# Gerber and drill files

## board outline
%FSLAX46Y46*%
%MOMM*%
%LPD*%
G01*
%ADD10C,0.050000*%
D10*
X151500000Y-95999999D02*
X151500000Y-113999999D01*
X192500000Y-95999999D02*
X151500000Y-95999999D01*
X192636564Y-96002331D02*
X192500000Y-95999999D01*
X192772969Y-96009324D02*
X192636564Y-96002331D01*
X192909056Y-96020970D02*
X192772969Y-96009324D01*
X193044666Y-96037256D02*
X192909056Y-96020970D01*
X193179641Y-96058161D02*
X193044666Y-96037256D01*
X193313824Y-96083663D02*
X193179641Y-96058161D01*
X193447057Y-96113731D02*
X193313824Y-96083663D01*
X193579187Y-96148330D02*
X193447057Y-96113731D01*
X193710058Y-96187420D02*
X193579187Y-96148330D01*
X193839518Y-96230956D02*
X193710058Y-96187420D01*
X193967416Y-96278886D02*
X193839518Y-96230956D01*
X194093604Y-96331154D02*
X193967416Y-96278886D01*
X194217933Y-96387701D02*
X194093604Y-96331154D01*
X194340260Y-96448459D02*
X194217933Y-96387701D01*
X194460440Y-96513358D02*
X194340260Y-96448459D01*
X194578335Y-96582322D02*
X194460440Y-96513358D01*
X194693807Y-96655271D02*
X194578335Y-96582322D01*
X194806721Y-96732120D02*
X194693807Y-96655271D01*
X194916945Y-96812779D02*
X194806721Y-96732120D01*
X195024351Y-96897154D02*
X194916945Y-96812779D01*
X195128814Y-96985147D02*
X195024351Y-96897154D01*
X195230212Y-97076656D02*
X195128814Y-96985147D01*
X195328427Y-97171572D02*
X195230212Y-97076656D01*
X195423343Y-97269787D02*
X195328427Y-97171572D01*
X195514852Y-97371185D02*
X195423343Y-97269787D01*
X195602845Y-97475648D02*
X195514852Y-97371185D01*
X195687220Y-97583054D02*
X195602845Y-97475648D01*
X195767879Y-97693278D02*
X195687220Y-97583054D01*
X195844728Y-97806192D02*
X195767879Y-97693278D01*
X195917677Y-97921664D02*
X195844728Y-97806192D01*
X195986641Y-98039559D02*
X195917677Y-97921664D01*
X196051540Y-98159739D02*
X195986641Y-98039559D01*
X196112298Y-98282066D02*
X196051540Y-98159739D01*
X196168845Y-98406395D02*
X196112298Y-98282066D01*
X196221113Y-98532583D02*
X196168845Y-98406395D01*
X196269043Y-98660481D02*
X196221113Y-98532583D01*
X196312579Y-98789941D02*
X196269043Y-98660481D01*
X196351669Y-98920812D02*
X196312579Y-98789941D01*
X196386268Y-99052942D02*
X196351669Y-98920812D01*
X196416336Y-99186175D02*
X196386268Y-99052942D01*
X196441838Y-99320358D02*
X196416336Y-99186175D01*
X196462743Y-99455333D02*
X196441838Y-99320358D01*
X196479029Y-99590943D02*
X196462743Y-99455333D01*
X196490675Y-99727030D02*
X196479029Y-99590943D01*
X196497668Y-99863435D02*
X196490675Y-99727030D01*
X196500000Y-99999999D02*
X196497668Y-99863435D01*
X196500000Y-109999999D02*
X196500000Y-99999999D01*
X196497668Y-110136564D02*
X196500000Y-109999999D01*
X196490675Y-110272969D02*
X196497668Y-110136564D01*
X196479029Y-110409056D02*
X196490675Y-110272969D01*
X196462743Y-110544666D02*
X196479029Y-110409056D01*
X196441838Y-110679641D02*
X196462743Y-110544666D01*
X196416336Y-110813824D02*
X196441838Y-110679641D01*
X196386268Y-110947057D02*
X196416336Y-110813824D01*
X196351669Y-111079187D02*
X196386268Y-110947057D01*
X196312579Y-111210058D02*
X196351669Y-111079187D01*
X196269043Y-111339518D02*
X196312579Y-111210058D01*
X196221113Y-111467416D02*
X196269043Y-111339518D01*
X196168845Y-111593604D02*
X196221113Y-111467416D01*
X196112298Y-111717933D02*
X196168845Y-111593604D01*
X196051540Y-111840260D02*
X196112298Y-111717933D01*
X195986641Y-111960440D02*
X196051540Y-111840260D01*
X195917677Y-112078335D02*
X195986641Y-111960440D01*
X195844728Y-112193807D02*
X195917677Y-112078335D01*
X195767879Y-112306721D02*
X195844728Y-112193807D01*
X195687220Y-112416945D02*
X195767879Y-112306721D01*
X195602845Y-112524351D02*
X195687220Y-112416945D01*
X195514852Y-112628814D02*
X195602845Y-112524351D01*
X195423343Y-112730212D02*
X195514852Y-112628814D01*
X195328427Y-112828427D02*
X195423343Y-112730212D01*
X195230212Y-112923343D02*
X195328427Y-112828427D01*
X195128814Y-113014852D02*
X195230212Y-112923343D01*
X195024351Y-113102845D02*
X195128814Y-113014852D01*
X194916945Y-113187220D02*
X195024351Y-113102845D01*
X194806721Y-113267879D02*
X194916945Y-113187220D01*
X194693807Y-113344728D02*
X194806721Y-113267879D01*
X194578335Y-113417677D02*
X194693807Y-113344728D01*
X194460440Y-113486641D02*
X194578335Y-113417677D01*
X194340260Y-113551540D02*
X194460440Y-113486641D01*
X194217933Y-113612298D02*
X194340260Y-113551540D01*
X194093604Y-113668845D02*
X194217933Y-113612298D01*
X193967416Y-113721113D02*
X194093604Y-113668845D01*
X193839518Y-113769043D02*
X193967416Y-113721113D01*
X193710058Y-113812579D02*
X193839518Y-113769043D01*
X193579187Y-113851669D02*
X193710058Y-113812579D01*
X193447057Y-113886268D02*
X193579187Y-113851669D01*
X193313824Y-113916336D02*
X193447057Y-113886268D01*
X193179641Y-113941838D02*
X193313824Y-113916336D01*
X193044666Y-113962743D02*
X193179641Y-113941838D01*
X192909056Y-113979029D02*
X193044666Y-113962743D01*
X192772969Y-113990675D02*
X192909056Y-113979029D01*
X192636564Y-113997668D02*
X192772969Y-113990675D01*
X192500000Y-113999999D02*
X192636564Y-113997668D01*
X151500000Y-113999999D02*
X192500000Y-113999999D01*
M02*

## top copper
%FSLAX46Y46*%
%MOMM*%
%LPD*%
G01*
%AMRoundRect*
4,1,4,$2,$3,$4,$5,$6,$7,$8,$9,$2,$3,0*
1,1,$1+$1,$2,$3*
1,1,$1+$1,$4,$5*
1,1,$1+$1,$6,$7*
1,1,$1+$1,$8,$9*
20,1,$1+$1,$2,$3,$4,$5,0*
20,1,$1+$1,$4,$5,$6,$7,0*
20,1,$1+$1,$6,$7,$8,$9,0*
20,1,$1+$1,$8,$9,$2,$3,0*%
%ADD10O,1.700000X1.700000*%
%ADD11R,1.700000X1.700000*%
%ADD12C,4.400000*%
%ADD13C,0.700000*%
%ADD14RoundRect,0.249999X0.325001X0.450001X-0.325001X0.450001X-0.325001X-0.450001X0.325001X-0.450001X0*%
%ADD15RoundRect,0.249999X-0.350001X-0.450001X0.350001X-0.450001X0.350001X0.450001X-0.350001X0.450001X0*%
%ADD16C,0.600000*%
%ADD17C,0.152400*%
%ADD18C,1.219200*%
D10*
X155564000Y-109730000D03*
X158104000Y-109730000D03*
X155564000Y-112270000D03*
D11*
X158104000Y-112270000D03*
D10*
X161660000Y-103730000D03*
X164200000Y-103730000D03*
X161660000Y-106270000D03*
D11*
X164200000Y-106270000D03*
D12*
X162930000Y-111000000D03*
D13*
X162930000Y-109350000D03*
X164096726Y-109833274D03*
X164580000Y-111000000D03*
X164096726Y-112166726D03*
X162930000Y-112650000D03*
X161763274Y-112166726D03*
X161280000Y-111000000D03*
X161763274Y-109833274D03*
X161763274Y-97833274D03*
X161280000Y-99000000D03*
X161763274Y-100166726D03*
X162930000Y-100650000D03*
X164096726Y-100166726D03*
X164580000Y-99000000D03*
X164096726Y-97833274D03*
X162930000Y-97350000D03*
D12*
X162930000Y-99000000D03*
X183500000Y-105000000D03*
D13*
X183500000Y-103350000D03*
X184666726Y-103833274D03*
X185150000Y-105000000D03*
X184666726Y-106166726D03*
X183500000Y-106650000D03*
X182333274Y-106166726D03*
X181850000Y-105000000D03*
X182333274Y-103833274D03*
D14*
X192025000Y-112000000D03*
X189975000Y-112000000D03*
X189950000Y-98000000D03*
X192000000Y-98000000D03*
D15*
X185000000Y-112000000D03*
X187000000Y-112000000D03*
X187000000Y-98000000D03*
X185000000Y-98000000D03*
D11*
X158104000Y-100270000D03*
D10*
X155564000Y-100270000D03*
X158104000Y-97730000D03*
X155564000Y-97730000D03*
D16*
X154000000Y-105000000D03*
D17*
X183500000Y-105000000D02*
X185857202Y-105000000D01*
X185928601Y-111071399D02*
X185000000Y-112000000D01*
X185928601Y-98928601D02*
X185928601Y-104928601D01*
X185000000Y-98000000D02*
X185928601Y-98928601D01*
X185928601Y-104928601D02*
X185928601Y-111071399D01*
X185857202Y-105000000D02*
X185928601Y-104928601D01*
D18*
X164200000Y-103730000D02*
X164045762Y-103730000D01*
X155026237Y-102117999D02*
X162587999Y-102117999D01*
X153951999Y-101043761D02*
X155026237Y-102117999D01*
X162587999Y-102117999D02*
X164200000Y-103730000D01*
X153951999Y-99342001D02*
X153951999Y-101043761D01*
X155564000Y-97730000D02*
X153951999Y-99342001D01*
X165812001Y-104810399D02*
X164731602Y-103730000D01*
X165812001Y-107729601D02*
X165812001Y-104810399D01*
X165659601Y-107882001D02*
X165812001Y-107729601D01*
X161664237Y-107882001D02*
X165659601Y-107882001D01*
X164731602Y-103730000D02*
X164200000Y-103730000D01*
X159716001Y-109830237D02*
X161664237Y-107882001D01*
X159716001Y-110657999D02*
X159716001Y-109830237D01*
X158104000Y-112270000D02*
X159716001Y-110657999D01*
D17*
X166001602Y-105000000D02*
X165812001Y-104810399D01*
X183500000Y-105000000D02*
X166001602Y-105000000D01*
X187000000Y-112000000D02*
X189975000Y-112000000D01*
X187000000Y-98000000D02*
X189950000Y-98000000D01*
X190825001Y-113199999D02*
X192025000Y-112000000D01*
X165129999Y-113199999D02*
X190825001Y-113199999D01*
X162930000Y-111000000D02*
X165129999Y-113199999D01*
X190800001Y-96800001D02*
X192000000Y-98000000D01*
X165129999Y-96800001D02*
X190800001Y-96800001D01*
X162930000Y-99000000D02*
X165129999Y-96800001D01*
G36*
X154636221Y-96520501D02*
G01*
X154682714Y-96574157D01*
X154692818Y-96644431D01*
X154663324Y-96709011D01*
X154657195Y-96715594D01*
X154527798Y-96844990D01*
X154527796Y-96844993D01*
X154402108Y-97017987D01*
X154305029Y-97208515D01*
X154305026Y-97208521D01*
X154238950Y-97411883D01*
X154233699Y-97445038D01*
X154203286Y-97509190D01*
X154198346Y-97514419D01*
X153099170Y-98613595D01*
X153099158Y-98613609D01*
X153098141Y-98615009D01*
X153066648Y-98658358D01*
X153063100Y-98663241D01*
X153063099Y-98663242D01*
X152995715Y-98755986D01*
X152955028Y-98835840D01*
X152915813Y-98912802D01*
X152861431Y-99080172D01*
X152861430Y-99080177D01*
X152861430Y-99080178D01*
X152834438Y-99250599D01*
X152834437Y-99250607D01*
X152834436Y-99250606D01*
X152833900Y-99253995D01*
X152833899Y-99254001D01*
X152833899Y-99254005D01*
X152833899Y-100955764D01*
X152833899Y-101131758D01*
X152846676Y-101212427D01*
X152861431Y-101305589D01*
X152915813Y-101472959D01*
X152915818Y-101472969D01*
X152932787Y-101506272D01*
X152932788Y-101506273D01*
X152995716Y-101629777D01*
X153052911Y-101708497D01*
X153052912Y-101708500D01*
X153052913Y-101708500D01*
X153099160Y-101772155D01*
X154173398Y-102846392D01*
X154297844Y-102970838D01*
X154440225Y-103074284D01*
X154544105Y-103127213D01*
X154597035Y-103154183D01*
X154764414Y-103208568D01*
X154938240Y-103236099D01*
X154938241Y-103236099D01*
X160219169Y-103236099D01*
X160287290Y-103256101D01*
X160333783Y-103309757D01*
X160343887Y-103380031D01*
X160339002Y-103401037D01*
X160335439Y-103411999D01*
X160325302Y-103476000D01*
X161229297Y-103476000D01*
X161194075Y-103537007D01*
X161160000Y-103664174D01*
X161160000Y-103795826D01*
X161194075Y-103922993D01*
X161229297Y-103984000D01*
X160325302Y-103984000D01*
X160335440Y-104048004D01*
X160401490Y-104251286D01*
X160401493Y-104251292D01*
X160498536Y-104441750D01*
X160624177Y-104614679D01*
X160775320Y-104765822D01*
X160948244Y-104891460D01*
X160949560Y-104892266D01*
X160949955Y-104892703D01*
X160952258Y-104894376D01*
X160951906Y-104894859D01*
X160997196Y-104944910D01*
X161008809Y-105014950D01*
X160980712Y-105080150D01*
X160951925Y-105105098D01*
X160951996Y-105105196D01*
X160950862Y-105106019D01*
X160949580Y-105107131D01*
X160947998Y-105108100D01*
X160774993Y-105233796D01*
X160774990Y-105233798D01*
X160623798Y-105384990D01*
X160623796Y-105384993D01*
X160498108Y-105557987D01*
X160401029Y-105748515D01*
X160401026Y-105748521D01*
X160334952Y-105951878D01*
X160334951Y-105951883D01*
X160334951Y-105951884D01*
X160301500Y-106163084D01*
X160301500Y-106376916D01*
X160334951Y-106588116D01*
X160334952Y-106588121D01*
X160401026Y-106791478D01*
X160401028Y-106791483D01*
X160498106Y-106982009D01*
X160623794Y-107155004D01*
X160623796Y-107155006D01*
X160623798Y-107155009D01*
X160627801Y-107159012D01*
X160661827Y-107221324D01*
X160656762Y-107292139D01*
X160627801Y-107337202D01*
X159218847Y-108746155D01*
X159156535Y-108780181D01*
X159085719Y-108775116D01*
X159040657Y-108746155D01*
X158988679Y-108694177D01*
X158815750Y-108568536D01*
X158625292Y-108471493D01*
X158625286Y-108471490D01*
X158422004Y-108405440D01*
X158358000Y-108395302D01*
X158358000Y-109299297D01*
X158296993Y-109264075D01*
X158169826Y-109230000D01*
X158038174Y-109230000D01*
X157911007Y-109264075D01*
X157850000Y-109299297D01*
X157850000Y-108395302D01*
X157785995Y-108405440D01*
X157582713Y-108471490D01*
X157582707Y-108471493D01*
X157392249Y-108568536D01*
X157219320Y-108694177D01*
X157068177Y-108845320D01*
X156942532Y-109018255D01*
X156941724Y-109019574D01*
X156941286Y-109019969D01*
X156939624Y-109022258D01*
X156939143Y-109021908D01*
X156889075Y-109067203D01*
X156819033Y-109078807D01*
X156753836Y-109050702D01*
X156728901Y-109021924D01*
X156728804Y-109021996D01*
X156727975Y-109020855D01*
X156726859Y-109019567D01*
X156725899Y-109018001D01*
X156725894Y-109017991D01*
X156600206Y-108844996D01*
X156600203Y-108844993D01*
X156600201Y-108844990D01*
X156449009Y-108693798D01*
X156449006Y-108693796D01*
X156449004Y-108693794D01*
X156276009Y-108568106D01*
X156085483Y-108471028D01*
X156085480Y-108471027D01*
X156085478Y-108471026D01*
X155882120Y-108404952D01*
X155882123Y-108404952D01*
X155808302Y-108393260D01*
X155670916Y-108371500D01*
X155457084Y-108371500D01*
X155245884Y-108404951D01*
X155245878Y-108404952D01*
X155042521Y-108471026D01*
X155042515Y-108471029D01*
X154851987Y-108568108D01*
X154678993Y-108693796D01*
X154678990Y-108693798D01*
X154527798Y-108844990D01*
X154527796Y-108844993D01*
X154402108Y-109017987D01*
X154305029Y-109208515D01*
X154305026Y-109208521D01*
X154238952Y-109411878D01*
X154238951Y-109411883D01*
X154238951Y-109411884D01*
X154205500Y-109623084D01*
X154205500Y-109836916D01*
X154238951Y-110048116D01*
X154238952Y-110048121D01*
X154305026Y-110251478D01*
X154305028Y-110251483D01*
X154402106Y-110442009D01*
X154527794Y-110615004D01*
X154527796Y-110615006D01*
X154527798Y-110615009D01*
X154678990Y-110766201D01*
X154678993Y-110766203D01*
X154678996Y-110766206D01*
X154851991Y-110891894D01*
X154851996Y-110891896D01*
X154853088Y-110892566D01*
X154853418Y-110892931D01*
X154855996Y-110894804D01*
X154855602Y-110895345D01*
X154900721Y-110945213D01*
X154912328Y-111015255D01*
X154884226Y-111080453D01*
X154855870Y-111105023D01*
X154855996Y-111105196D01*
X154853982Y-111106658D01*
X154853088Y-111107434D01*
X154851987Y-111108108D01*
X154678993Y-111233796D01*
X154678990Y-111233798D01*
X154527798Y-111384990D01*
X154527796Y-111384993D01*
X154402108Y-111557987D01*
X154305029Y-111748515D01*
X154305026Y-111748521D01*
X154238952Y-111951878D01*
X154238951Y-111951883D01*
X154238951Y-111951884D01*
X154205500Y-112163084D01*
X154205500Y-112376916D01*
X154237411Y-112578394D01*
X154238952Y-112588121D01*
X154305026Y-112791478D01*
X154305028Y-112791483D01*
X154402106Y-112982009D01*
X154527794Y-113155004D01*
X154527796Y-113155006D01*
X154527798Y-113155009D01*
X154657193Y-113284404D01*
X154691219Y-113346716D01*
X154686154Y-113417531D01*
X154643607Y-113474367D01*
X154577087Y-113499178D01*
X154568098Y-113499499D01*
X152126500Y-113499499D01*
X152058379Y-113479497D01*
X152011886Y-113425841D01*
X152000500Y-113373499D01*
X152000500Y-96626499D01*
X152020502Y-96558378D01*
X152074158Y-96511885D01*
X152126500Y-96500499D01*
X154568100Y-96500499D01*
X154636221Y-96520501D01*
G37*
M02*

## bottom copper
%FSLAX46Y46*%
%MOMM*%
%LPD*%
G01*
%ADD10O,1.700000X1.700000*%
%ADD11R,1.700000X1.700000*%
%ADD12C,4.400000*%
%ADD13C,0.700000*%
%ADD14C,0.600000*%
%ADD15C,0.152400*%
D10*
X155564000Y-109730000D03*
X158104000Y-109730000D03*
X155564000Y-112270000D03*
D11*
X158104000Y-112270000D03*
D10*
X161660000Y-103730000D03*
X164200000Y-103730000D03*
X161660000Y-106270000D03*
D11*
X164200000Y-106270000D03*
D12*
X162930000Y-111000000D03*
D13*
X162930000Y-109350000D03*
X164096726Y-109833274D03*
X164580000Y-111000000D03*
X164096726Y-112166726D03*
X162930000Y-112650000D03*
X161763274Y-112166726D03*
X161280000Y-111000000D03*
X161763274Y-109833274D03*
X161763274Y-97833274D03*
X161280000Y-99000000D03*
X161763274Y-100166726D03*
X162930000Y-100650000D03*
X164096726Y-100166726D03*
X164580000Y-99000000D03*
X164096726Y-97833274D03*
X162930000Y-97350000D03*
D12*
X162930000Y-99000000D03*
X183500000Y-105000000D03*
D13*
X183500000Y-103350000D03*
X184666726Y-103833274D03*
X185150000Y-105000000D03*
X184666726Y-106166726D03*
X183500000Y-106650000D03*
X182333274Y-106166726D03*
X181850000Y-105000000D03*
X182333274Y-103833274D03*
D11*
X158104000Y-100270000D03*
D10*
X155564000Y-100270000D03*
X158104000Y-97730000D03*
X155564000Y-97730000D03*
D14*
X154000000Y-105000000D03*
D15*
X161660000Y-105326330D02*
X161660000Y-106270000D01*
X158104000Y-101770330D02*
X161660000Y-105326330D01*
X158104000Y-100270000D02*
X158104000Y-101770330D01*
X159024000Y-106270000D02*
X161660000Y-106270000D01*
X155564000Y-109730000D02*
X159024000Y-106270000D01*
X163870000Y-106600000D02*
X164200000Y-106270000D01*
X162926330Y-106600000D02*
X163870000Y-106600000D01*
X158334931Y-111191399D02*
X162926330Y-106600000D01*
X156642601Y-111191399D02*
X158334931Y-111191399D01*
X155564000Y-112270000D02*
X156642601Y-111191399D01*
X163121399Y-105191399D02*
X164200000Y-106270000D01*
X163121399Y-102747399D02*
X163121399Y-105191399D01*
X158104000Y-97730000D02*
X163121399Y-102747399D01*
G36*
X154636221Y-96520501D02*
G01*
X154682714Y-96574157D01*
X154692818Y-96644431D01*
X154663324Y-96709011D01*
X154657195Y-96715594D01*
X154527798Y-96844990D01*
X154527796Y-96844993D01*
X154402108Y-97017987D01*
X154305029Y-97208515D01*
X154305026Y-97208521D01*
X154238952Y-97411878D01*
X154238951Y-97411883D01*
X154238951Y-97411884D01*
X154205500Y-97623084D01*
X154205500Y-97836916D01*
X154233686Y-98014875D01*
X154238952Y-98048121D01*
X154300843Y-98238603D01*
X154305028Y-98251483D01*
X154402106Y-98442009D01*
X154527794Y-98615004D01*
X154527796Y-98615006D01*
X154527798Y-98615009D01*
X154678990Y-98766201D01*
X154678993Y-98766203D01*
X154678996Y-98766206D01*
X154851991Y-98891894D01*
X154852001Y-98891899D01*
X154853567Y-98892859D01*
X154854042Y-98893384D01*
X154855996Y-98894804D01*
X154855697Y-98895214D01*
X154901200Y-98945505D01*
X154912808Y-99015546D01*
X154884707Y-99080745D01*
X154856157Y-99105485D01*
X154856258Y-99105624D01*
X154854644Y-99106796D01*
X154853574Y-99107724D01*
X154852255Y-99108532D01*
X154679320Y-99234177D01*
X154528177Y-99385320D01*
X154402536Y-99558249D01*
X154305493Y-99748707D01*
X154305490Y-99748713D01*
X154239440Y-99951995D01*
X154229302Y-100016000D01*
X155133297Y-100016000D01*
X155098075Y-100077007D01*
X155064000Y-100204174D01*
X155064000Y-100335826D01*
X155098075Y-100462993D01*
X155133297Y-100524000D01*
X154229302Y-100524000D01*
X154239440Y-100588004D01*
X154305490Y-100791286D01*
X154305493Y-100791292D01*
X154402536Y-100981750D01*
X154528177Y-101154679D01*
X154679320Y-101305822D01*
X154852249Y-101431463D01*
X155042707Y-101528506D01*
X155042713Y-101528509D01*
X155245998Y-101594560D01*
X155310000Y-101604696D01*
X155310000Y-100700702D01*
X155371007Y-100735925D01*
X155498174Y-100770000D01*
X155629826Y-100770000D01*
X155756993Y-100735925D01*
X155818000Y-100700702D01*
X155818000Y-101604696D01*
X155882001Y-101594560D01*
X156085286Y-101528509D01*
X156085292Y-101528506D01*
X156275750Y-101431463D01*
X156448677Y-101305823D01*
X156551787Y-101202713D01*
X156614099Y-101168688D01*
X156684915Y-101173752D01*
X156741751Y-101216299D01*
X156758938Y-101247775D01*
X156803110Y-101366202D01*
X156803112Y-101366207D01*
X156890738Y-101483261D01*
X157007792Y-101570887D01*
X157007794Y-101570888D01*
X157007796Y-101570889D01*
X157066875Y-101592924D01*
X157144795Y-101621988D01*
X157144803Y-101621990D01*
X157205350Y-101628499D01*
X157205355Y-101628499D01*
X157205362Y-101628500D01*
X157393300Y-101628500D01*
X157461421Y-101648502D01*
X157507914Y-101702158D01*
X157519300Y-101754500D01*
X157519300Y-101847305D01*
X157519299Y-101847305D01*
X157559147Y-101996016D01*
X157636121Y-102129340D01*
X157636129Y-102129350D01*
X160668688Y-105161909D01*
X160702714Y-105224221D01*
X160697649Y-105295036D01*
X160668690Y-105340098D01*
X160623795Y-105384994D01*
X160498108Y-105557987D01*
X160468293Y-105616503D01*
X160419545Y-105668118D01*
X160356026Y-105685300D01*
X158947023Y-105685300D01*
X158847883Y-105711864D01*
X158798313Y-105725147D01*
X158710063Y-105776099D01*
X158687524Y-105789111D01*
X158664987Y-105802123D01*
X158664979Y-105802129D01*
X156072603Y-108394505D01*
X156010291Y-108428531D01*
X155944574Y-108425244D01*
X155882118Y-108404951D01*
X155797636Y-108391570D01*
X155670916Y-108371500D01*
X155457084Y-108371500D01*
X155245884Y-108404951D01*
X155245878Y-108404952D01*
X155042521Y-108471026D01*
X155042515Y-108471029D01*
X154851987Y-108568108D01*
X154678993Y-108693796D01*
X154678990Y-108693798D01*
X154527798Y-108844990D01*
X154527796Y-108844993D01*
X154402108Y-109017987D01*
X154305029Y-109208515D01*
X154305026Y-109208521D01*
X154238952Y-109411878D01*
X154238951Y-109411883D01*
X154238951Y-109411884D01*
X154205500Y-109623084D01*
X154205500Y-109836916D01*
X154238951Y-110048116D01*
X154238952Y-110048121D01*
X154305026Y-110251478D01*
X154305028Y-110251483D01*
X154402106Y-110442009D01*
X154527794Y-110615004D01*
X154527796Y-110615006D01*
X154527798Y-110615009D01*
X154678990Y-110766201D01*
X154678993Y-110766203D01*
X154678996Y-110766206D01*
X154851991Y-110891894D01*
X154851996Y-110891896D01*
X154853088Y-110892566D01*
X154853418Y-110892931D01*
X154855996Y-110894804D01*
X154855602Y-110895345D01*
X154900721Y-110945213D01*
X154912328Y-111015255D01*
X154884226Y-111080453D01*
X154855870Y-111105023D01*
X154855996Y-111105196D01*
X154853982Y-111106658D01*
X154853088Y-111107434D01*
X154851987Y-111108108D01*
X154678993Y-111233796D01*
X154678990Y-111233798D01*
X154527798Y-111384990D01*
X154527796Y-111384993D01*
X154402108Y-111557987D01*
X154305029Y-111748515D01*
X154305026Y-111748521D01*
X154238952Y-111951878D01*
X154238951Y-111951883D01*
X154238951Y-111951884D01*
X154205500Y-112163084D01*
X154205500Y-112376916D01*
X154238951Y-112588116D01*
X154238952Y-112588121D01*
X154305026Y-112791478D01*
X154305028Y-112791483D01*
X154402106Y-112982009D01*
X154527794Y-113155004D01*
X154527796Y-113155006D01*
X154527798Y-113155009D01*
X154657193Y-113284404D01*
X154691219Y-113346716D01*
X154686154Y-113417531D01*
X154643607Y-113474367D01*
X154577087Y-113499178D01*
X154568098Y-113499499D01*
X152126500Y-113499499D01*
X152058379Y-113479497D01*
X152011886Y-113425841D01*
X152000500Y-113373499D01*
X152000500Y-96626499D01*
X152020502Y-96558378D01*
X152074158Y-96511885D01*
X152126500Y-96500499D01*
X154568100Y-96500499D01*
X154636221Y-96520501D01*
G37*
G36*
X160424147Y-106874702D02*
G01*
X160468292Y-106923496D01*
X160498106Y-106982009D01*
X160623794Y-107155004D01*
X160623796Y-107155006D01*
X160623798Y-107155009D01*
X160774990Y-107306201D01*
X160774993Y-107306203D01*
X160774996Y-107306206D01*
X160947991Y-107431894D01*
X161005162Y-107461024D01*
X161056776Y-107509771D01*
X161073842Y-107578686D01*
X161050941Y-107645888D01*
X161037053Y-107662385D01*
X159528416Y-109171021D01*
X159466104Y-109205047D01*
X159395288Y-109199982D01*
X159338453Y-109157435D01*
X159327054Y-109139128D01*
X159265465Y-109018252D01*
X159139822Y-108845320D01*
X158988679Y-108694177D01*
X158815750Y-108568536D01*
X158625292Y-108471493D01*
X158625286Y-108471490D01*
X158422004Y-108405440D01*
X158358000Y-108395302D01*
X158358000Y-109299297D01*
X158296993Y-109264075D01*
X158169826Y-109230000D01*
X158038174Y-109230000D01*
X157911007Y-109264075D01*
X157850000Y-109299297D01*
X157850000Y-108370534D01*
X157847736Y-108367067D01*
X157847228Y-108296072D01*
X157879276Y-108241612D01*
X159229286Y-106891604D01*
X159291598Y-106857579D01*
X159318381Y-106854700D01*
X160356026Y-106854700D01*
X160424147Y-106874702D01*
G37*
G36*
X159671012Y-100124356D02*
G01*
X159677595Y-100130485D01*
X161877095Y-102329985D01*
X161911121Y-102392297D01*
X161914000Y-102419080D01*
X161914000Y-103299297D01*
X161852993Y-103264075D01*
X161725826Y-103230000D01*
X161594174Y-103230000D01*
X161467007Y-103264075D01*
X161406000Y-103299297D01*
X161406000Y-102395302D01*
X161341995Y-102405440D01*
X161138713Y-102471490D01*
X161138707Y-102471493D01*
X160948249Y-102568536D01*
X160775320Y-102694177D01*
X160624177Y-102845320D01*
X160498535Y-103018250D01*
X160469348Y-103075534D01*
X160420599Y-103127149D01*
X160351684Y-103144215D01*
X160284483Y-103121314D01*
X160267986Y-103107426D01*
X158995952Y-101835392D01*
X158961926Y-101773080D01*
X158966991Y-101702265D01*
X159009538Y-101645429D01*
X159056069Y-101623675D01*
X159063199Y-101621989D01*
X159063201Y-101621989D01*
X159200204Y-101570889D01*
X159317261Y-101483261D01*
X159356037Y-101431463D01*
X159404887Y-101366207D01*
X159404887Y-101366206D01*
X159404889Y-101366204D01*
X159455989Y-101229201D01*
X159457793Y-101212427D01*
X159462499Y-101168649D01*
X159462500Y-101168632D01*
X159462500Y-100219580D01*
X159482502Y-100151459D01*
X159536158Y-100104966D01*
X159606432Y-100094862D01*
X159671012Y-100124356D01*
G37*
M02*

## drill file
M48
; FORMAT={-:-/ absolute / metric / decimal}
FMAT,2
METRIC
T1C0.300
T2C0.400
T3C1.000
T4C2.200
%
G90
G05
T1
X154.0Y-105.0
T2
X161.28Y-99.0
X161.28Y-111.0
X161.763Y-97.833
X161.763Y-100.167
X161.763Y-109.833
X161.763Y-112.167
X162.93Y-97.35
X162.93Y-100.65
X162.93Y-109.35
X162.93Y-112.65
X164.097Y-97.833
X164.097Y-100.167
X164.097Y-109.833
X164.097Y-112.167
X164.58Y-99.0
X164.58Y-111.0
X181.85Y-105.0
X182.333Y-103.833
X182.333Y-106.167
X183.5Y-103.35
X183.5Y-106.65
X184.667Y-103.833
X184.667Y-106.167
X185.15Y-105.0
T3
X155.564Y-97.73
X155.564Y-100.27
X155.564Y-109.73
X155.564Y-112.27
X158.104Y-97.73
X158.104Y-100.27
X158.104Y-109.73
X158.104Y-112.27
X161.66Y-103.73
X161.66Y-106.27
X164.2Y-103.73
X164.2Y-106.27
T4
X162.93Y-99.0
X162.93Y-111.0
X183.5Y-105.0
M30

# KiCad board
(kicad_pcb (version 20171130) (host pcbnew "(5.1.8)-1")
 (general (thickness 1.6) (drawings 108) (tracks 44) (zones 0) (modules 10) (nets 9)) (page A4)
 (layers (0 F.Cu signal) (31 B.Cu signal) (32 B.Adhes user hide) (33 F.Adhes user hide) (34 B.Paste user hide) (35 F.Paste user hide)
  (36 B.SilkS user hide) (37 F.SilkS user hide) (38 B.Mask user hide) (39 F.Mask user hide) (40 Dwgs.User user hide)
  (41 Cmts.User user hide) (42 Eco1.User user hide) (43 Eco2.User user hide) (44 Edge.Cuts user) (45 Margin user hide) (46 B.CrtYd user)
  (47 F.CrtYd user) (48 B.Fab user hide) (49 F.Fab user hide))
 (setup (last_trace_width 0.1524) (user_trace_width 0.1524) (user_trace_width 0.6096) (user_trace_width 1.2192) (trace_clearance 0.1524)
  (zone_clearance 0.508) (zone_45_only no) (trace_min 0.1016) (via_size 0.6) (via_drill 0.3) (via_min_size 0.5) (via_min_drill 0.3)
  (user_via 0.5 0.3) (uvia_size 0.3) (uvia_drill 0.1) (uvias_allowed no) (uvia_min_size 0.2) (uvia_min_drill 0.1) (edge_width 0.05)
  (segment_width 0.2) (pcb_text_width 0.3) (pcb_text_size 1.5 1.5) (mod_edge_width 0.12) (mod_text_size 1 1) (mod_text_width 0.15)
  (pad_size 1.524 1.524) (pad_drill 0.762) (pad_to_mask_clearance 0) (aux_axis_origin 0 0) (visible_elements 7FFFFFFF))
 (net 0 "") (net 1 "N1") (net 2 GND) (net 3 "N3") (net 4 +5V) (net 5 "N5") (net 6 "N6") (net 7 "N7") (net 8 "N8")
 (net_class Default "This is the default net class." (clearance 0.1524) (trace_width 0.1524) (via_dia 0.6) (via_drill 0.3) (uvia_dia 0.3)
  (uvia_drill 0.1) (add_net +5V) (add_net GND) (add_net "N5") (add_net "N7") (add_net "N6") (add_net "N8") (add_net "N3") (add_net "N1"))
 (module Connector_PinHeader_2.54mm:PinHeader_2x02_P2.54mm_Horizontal (layer F.Cu) (at 158.104 112.27 180)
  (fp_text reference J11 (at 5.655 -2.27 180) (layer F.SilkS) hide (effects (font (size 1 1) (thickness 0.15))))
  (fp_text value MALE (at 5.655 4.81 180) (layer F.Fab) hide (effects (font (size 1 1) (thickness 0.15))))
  (pad 4 thru_hole oval (at 2.54 2.54 180) (size 1.7 1.7) (drill 1) (layers *.Cu *.Mask) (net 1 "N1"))
  (pad 3 thru_hole oval (at 0 2.54 180) (size 1.7 1.7) (drill 1) (layers *.Cu *.Mask) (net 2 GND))
  (pad 2 thru_hole oval (at 2.54 0 180) (size 1.7 1.7) (drill 1) (layers *.Cu *.Mask) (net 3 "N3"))
  (pad 1 thru_hole rect (at 0 0 180) (size 1.7 1.7) (drill 1) (layers *.Cu *.Mask) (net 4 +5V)))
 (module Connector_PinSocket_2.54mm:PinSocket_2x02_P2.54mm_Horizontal (layer B.Cu) (at 164.2 106.27)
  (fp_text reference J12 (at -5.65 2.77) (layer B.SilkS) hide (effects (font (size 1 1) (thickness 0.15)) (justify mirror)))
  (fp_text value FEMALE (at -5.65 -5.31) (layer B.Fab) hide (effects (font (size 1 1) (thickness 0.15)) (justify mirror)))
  (pad 4 thru_hole oval (at -2.54 -2.54) (size 1.7 1.7) (drill 1) (layers *.Cu *.Mask) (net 2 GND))
  (pad 3 thru_hole oval (at 0 -2.54) (size 1.7 1.7) (drill 1) (layers *.Cu *.Mask) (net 4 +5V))
  (pad 2 thru_hole oval (at -2.54 0) (size 1.7 1.7) (drill 1) (layers *.Cu *.Mask) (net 1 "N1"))
  (pad 1 thru_hole rect (at 0 0) (size 1.7 1.7) (drill 1) (layers *.Cu *.Mask) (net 3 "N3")))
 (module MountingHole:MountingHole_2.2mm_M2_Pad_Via (layer F.Cu) (at 162.93 111 90)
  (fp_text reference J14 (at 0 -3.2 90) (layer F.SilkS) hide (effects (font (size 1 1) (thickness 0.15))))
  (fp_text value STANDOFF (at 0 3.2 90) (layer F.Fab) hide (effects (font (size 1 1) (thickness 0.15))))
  (pad 1 thru_hole circle (at 0 0 90) (size 4.4 4.4) (drill 2.2) (layers *.Cu *.Mask) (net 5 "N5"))
  (pad 1 thru_hole circle (at 1.65 0 90) (size 0.7 0.7) (drill 0.4) (layers *.Cu *.Mask) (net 5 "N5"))
  (pad 1 thru_hole circle (at 1.166726 1.166726 90) (size 0.7 0.7) (drill 0.4) (layers *.Cu *.Mask) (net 5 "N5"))
  (pad 1 thru_hole circle (at 0 1.65 90) (size 0.7 0.7) (drill 0.4) (layers *.Cu *.Mask) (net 5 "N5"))
  (pad 1 thru_hole circle (at -1.166726 1.166726 90) (size 0.7 0.7) (drill 0.4) (layers *.Cu *.Mask) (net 5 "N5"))
  (pad 1 thru_hole circle (at -1.65 0 90) (size 0.7 0.7) (drill 0.4) (layers *.Cu *.Mask) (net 5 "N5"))
  (pad 1 thru_hole circle (at -1.166726 -1.166726 90) (size 0.7 0.7) (drill 0.4) (layers *.Cu *.Mask) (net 5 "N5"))
  (pad 1 thru_hole circle (at 0 -1.65 90) (size 0.7 0.7) (drill 0.4) (layers *.Cu *.Mask) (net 5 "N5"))
  (pad 1 thru_hole circle (at 1.166726 -1.166726 90) (size 0.7 0.7) (drill 0.4) (layers *.Cu *.Mask) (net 5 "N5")))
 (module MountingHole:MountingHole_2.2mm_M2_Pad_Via (layer F.Cu) (at 162.93 99 90)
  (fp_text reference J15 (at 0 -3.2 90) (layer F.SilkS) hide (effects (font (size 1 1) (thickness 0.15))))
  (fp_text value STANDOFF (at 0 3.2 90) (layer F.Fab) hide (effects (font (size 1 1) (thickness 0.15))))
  (pad 1 thru_hole circle (at 1.166726 -1.166726 90) (size 0.7 0.7) (drill 0.4) (layers *.Cu *.Mask) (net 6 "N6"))
  (pad 1 thru_hole circle (at 0 -1.65 90) (size 0.7 0.7) (drill 0.4) (layers *.Cu *.Mask) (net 6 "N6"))
  (pad 1 thru_hole circle (at -1.166726 -1.166726 90) (size 0.7 0.7) (drill 0.4) (layers *.Cu *.Mask) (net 6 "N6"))
  (pad 1 thru_hole circle (at -1.65 0 90) (size 0.7 0.7) (drill 0.4) (layers *.Cu *.Mask) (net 6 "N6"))
  (pad 1 thru_hole circle (at -1.166726 1.166726 90) (size 0.7 0.7) (drill 0.4) (layers *.Cu *.Mask) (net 6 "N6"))
  (pad 1 thru_hole circle (at 0 1.65 90) (size 0.7 0.7) (drill 0.4) (layers *.Cu *.Mask) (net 6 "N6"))
  (pad 1 thru_hole circle (at 1.166726 1.166726 90) (size 0.7 0.7) (drill 0.4) (layers *.Cu *.Mask) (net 6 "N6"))
  (pad 1 thru_hole circle (at 1.65 0 90) (size 0.7 0.7) (drill 0.4) (layers *.Cu *.Mask) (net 6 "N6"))
  (pad 1 thru_hole circle (at 0 0 90) (size 4.4 4.4) (drill 2.2) (layers *.Cu *.Mask) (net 6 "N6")))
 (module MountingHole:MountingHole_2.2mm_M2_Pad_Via (layer F.Cu) (at 183.5 105 90)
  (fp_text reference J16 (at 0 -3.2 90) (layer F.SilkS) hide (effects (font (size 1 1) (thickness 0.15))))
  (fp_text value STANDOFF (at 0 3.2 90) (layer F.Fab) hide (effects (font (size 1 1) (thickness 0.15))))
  (pad 1 thru_hole circle (at 0 0 90) (size 4.4 4.4) (drill 2.2) (layers *.Cu *.Mask) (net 4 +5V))
  (pad 1 thru_hole circle (at 1.65 0 90) (size 0.7 0.7) (drill 0.4) (layers *.Cu *.Mask) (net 4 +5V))
  (pad 1 thru_hole circle (at 1.166726 1.166726 90) (size 0.7 0.7) (drill 0.4) (layers *.Cu *.Mask) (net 4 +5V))
  (pad 1 thru_hole circle (at 0 1.65 90) (size 0.7 0.7) (drill 0.4) (layers *.Cu *.Mask) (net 4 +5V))
  (pad 1 thru_hole circle (at -1.166726 1.166726 90) (size 0.7 0.7) (drill 0.4) (layers *.Cu *.Mask) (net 4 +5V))
  (pad 1 thru_hole circle (at -1.65 0 90) (size 0.7 0.7) (drill 0.4) (layers *.Cu *.Mask) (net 4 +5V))
  (pad 1 thru_hole circle (at -1.166726 -1.166726 90) (size 0.7 0.7) (drill 0.4) (layers *.Cu *.Mask) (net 4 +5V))
  (pad 1 thru_hole circle (at 0 -1.65 90) (size 0.7 0.7) (drill 0.4) (layers *.Cu *.Mask) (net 4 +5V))
  (pad 1 thru_hole circle (at 1.166726 -1.166726 90) (size 0.7 0.7) (drill 0.4) (layers *.Cu *.Mask) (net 4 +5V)))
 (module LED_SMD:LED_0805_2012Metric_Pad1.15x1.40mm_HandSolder (layer F.Cu) (at 191 112 180)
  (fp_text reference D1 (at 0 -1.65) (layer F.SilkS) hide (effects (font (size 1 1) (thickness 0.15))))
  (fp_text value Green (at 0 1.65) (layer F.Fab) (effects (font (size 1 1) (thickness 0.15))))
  (pad 1 smd roundrect (at -1.025 0 180) (size 1.15 1.4) (layers F.Cu F.Paste F.Mask) (roundrect_rratio 0.2173904347826087) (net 5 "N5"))
  (pad 2 smd roundrect (at 1.025 0 180) (size 1.15 1.4) (layers F.Cu F.Paste F.Mask) (roundrect_rratio 0.2173904347826087) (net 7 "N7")))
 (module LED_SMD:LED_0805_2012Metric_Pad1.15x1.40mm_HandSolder (layer F.Cu) (at 190.975 98 180)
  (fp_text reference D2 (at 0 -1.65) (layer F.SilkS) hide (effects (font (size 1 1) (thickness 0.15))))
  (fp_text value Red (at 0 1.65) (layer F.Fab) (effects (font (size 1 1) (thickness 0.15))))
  (pad 2 smd roundrect (at 1.025 0 180) (size 1.15 1.4) (layers F.Cu F.Paste F.Mask) (roundrect_rratio 0.2173904347826087) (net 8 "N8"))
  (pad 1 smd roundrect (at -1.025 0 180) (size 1.15 1.4) (layers F.Cu F.Paste F.Mask) (roundrect_rratio 0.2173904347826087) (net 6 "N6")))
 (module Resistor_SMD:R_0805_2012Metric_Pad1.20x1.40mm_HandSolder (layer F.Cu) (at 186 112)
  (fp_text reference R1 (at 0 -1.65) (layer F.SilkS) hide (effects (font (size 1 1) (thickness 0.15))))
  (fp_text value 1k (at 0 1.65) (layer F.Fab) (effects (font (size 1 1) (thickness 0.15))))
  (pad 1 smd roundrect (at -1 0) (size 1.2 1.4) (layers F.Cu F.Paste F.Mask) (roundrect_rratio 0.2083325) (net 4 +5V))
  (pad 2 smd roundrect (at 1 0) (size 1.2 1.4) (layers F.Cu F.Paste F.Mask) (roundrect_rratio 0.2083325) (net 7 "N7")))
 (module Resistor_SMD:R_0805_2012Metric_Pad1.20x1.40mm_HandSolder (layer F.Cu) (at 186 98)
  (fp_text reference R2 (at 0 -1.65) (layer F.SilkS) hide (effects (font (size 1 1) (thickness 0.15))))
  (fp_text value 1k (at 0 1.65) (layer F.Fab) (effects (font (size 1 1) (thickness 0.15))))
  (pad 2 smd roundrect (at 1 0) (size 1.2 1.4) (layers F.Cu F.Paste F.Mask) (roundrect_rratio 0.2083325) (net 8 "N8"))
  (pad 1 smd roundrect (at -1 0) (size 1.2 1.4) (layers F.Cu F.Paste F.Mask) (roundrect_rratio 0.2083325) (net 4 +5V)))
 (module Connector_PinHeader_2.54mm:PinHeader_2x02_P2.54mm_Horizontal (layer F.Cu) (at 158.104 100.27 180)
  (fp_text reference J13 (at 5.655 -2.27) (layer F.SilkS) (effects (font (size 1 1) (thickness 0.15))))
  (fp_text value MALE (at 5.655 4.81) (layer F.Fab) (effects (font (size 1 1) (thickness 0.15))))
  (pad 1 thru_hole rect (at 0 0 180) (size 1.7 1.7) (drill 1) (layers *.Cu *.Mask) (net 1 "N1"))
  (pad 2 thru_hole oval (at 2.54 0 180) (size 1.7 1.7) (drill 1) (layers *.Cu *.Mask) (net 2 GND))
  (pad 3 thru_hole oval (at 0 2.54 180) (size 1.7 1.7) (drill 1) (layers *.Cu *.Mask) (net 3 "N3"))
  (pad 4 thru_hole oval (at 2.54 2.54 180) (size 1.7 1.7) (drill 1) (layers *.Cu *.Mask) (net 4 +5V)))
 (gr_line (start 151.5 95.999999) (end 151.5 113.999999) (layer Edge.Cuts) (width 0.05))
 (gr_line (start 192.5 95.999999) (end 151.5 95.999999) (layer Edge.Cuts) (width 0.05))
 (gr_line (start 192.636564 96.002331) (end 192.5 95.999999) (layer Edge.Cuts) (width 0.05))
 (gr_line (start 192.772969 96.009324) (end 192.636564 96.002331) (layer Edge.Cuts) (width 0.05))
 (gr_line (start 192.909056 96.02097) (end 192.772969 96.009324) (layer Edge.Cuts) (width 0.05))
 (gr_line (start 193.044666 96.037256) (end 192.909056 96.02097) (layer Edge.Cuts) (width 0.05))
 (gr_line (start 193.179641 96.058161) (end 193.044666 96.037256) (layer Edge.Cuts) (width 0.05))
 (gr_line (start 193.313824 96.083663) (end 193.179641 96.058161) (layer Edge.Cuts) (width 0.05))
 (gr_line (start 193.447057 96.113731) (end 193.313824 96.083663) (layer Edge.Cuts) (width 0.05))
 (gr_line (start 193.579187 96.14833) (end 193.447057 96.113731) (layer Edge.Cuts) (width 0.05))
 (gr_line (start 193.710058 96.18742) (end 193.579187 96.14833) (layer Edge.Cuts) (width 0.05))
 (gr_line (start 193.839518 96.230956) (end 193.710058 96.18742) (layer Edge.Cuts) (width 0.05))
 (gr_line (start 193.967416 96.278886) (end 193.839518 96.230956) (layer Edge.Cuts) (width 0.05))
 (gr_line (start 194.093604 96.331154) (end 193.967416 96.278886) (layer Edge.Cuts) (width 0.05))
 (gr_line (start 194.217933 96.387701) (end 194.093604 96.331154) (layer Edge.Cuts) (width 0.05))
 (gr_line (start 194.34026 96.448459) (end 194.217933 96.387701) (layer Edge.Cuts) (width 0.05))
 (gr_line (start 194.46044 96.513358) (end 194.34026 96.448459) (layer Edge.Cuts) (width 0.05))
 (gr_line (start 194.578335 96.582322) (end 194.46044 96.513358) (layer Edge.Cuts) (width 0.05))
 (gr_line (start 194.693807 96.655271) (end 194.578335 96.582322) (layer Edge.Cuts) (width 0.05))
 (gr_line (start 194.806721 96.73212) (end 194.693807 96.655271) (layer Edge.Cuts) (width 0.05))
 (gr_line (start 194.916945 96.812779) (end 194.806721 96.73212) (layer Edge.Cuts) (width 0.05))
 (gr_line (start 195.024351 96.897154) (end 194.916945 96.812779) (layer Edge.Cuts) (width 0.05))
 (gr_line (start 195.128814 96.985147) (end 195.024351 96.897154) (layer Edge.Cuts) (width 0.05))
 (gr_line (start 195.230212 97.076656) (end 195.128814 96.985147) (layer Edge.Cuts) (width 0.05))
 (gr_line (start 195.328427 97.171572) (end 195.230212 97.076656) (layer Edge.Cuts) (width 0.05))
 (gr_line (start 195.423343 97.269787) (end 195.328427 97.171572) (layer Edge.Cuts) (width 0.05))
 (gr_line (start 195.514852 97.371185) (end 195.423343 97.269787) (layer Edge.Cuts) (width 0.05))
 (gr_line (start 195.602845 97.475648) (end 195.514852 97.371185) (layer Edge.Cuts) (width 0.05))
 (gr_line (start 195.68722 97.583054) (end 195.602845 97.475648) (layer Edge.Cuts) (width 0.05))
 (gr_line (start 195.767879 97.693278) (end 195.68722 97.583054) (layer Edge.Cuts) (width 0.05))
 (gr_line (start 195.844728 97.806192) (end 195.767879 97.693278) (layer Edge.Cuts) (width 0.05))
 (gr_line (start 195.917677 97.921664) (end 195.844728 97.806192) (layer Edge.Cuts) (width 0.05))
 (gr_line (start 195.986641 98.039559) (end 195.917677 97.921664) (layer Edge.Cuts) (width 0.05))
 (gr_line (start 196.05154 98.159739) (end 195.986641 98.039559) (layer Edge.Cuts) (width 0.05))
 (gr_line (start 196.112298 98.282066) (end 196.05154 98.159739) (layer Edge.Cuts) (width 0.05))
 (gr_line (start 196.168845 98.406395) (end 196.112298 98.282066) (layer Edge.Cuts) (width 0.05))
 (gr_line (start 196.221113 98.532583) (end 196.168845 98.406395) (layer Edge.Cuts) (width 0.05))
 (gr_line (start 196.269043 98.660481) (end 196.221113 98.532583) (layer Edge.Cuts) (width 0.05))
 (gr_line (start 196.312579 98.789941) (end 196.269043 98.660481) (layer Edge.Cuts) (width 0.05))
 (gr_line (start 196.351669 98.920812) (end 196.312579 98.789941) (layer Edge.Cuts) (width 0.05))
 (gr_line (start 196.386268 99.052942) (end 196.351669 98.920812) (layer Edge.Cuts) (width 0.05))
 (gr_line (start 196.416336 99.186175) (end 196.386268 99.052942) (layer Edge.Cuts) (width 0.05))
 (gr_line (start 196.441838 99.320358) (end 196.416336 99.186175) (layer Edge.Cuts) (width 0.05))
 (gr_line (start 196.462743 99.455333) (end 196.441838 99.320358) (layer Edge.Cuts) (width 0.05))
 (gr_line (start 196.479029 99.590943) (end 196.462743 99.455333) (layer Edge.Cuts) (width 0.05))
 (gr_line (start 196.490675 99.72703) (end 196.479029 99.590943) (layer Edge.Cuts) (width 0.05))
 (gr_line (start 196.497668 99.863435) (end 196.490675 99.72703) (layer Edge.Cuts) (width 0.05))
 (gr_line (start 196.5 99.999999) (end 196.497668 99.863435) (layer Edge.Cuts) (width 0.05))
 (gr_line (start 196.5 109.999999) (end 196.5 99.999999) (layer Edge.Cuts) (width 0.05))
 (gr_line (start 196.497668 110.136564) (end 196.5 109.999999) (layer Edge.Cuts) (width 0.05))
 (gr_line (start 196.490675 110.272969) (end 196.497668 110.136564) (layer Edge.Cuts) (width 0.05))
 (gr_line (start 196.479029 110.409056) (end 196.490675 110.272969) (layer Edge.Cuts) (width 0.05))
 (gr_line (start 196.462743 110.544666) (end 196.479029 110.409056) (layer Edge.Cuts) (width 0.05))
 (gr_line (start 196.441838 110.679641) (end 196.462743 110.544666) (layer Edge.Cuts) (width 0.05))
 (gr_line (start 196.416336 110.813824) (end 196.441838 110.679641) (layer Edge.Cuts) (width 0.05))
 (gr_line (start 196.386268 110.947057) (end 196.416336 110.813824) (layer Edge.Cuts) (width 0.05))
 (gr_line (start 196.351669 111.079187) (end 196.386268 110.947057) (layer Edge.Cuts) (width 0.05))
 (gr_line (start 196.312579 111.210058) (end 196.351669 111.079187) (layer Edge.Cuts) (width 0.05))
 (gr_line (start 196.269043 111.339518) (end 196.312579 111.210058) (layer Edge.Cuts) (width 0.05))
 (gr_line (start 196.221113 111.467416) (end 196.269043 111.339518) (layer Edge.Cuts) (width 0.05))
 (gr_line (start 196.168845 111.593604) (end 196.221113 111.467416) (layer Edge.Cuts) (width 0.05))
 (gr_line (start 196.112298 111.717933) (end 196.168845 111.593604) (layer Edge.Cuts) (width 0.05))
 (gr_line (start 196.05154 111.84026) (end 196.112298 111.717933) (layer Edge.Cuts) (width 0.05))
 (gr_line (start 195.986641 111.96044) (end 196.05154 111.84026) (layer Edge.Cuts) (width 0.05))
 (gr_line (start 195.917677 112.078335) (end 195.986641 111.96044) (layer Edge.Cuts) (width 0.05))
 (gr_line (start 195.844728 112.193807) (end 195.917677 112.078335) (layer Edge.Cuts) (width 0.05))
 (gr_line (start 195.767879 112.306721) (end 195.844728 112.193807) (layer Edge.Cuts) (width 0.05))
 (gr_line (start 195.68722 112.416945) (end 195.767879 112.306721) (layer Edge.Cuts) (width 0.05))
 (gr_line (start 195.602845 112.524351) (end 195.68722 112.416945) (layer Edge.Cuts) (width 0.05))
 (gr_line (start 195.514852 112.628814) (end 195.602845 112.524351) (layer Edge.Cuts) (width 0.05))
 (gr_line (start 195.423343 112.730212) (end 195.514852 112.628814) (layer Edge.Cuts) (width 0.05))
 (gr_line (start 195.328427 112.828427) (end 195.423343 112.730212) (layer Edge.Cuts) (width 0.05))
 (gr_line (start 195.230212 112.923343) (end 195.328427 112.828427) (layer Edge.Cuts) (width 0.05))
 (gr_line (start 195.128814 113.014852) (end 195.230212 112.923343) (layer Edge.Cuts) (width 0.05))
 (gr_line (start 195.024351 113.102845) (end 195.128814 113.014852) (layer Edge.Cuts) (width 0.05))
 (gr_line (start 194.916945 113.18722) (end 195.024351 113.102845) (layer Edge.Cuts) (width 0.05))
 (gr_line (start 194.806721 113.267879) (end 194.916945 113.18722) (layer Edge.Cuts) (width 0.05))
 (gr_line (start 194.693807 113.344728) (end 194.806721 113.267879) (layer Edge.Cuts) (width 0.05))
 (gr_line (start 194.578335 113.417677) (end 194.693807 113.344728) (layer Edge.Cuts) (width 0.05))
 (gr_line (start 194.46044 113.486641) (end 194.578335 113.417677) (layer Edge.Cuts) (width 0.05))
 (gr_line (start 194.34026 113.55154) (end 194.46044 113.486641) (layer Edge.Cuts) (width 0.05))
 (gr_line (start 194.217933 113.612298) (end 194.34026 113.55154) (layer Edge.Cuts) (width 0.05))
 (gr_line (start 194.093604 113.668845) (end 194.217933 113.612298) (layer Edge.Cuts) (width 0.05))
 (gr_line (start 193.967416 113.721113) (end 194.093604 113.668845) (layer Edge.Cuts) (width 0.05))
 (gr_line (start 193.839518 113.769043) (end 193.967416 113.721113) (layer Edge.Cuts) (width 0.05))
 (gr_line (start 193.710058 113.812579) (end 193.839518 113.769043) (layer Edge.Cuts) (width 0.05))
 (gr_line (start 193.579187 113.851669) (end 193.710058 113.812579) (layer Edge.Cuts) (width 0.05))
 (gr_line (start 193.447057 113.886268) (end 193.579187 113.851669) (layer Edge.Cuts) (width 0.05))
 (gr_line (start 193.313824 113.916336) (end 193.447057 113.886268) (layer Edge.Cuts) (width 0.05))
 (gr_line (start 193.179641 113.941838) (end 193.313824 113.916336) (layer Edge.Cuts) (width 0.05))
 (gr_line (start 193.044666 113.962743) (end 193.179641 113.941838) (layer Edge.Cuts) (width 0.05))
 (gr_line (start 192.909056 113.979029) (end 193.044666 113.962743) (layer Edge.Cuts) (width 0.05))
 (gr_line (start 192.772969 113.990675) (end 192.909056 113.979029) (layer Edge.Cuts) (width 0.05))
 (gr_line (start 192.636564 113.997668) (end 192.772969 113.990675) (layer Edge.Cuts) (width 0.05))
 (gr_line (start 192.5 113.999999) (end 192.636564 113.997668) (layer Edge.Cuts) (width 0.05))
 (gr_line (start 151.5 113.999999) (end 192.5 113.999999) (layer Edge.Cuts) (width 0.05))
 (via (at 154 105) (size 0.6) (drill 0.3) (layers F.Cu B.Cu) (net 2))
 (segment (start 183.5 105) (end 185.857202 105) (width 0.1524) (layer F.Cu) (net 4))
 (segment (start 185.928601 111.071399) (end 185 112) (width 0.1524) (layer F.Cu) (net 4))
 (segment (start 185.928601 98.928601) (end 185.928601 104.928601) (width 0.1524) (layer F.Cu) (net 4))
 (segment (start 185 98) (end 185.928601 98.928601) (width 0.1524) (layer F.Cu) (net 4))
 (segment (start 185.928601 104.928601) (end 185.928601 111.071399) (width 0.1524) (layer F.Cu) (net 4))
 (segment (start 185.857202 105) (end 185.928601 104.928601) (width 0.1524) (layer F.Cu) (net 4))
 (segment (start 164.2 103.73) (end 164.045762 103.73) (width 1.2192) (layer F.Cu) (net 4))
 (segment (start 155.026237 102.117999) (end 162.587999 102.117999) (width 1.2192) (layer F.Cu) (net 4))
 (segment (start 153.951999 101.043761) (end 155.026237 102.117999) (width 1.2192) (layer F.Cu) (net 4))
 (segment (start 162.587999 102.117999) (end 164.2 103.73) (width 1.2192) (layer F.Cu) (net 4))
 (segment (start 153.951999 99.342001) (end 153.951999 101.043761) (width 1.2192) (layer F.Cu) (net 4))
 (segment (start 155.564 97.73) (end 153.951999 99.342001) (width 1.2192) (layer F.Cu) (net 4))
 (segment (start 165.812001 104.810399) (end 164.731602 103.73) (width 1.2192) (layer F.Cu) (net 4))
 (segment (start 165.812001 107.729601) (end 165.812001 104.810399) (width 1.2192) (layer F.Cu) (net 4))
 (segment (start 165.659601 107.882001) (end 165.812001 107.729601) (width 1.2192) (layer F.Cu) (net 4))
 (segment (start 161.664237 107.882001) (end 165.659601 107.882001) (width 1.2192) (layer F.Cu) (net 4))
 (segment (start 164.731602 103.73) (end 164.2 103.73) (width 1.2192) (layer F.Cu) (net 4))
 (segment (start 159.716001 109.830237) (end 161.664237 107.882001) (width 1.2192) (layer F.Cu) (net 4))
 (segment (start 159.716001 110.657999) (end 159.716001 109.830237) (width 1.2192) (layer F.Cu) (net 4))
 (segment (start 158.104 112.27) (end 159.716001 110.657999) (width 1.2192) (layer F.Cu) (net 4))
 (segment (start 166.001602 105) (end 165.812001 104.810399) (width 0.1524) (layer F.Cu) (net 4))
 (segment (start 183.5 105) (end 166.001602 105) (width 0.1524) (layer F.Cu) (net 4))
 (segment (start 187 112) (end 189.975 112) (width 0.1524) (layer F.Cu) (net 7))
 (segment (start 187 98) (end 189.95 98) (width 0.1524) (layer F.Cu) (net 8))
 (segment (start 161.66 105.32633) (end 161.66 106.27) (width 0.1524) (layer B.Cu) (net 1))
 (segment (start 158.104 101.77033) (end 161.66 105.32633) (width 0.1524) (layer B.Cu) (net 1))
 (segment (start 158.104 100.27) (end 158.104 101.77033) (width 0.1524) (layer B.Cu) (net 1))
 (segment (start 159.024 106.27) (end 161.66 106.27) (width 0.1524) (layer B.Cu) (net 1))
 (segment (start 155.564 109.73) (end 159.024 106.27) (width 0.1524) (layer B.Cu) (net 1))
 (segment (start 163.87 106.6) (end 164.2 106.27) (width 0.1524) (layer B.Cu) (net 3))
 (segment (start 162.92633 106.6) (end 163.87 106.6) (width 0.1524) (layer B.Cu) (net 3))
 (segment (start 158.334931 111.191399) (end 162.92633 106.6) (width 0.1524) (layer B.Cu) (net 3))
 (segment (start 156.642601 111.191399) (end 158.334931 111.191399) (width 0.1524) (layer B.Cu) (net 3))
 (segment (start 155.564 112.27) (end 156.642601 111.191399) (width 0.1524) (layer B.Cu) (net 3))
 (segment (start 163.121399 105.191399) (end 164.2 106.27) (width 0.1524) (layer B.Cu) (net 3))
 (segment (start 163.121399 102.747399) (end 163.121399 105.191399) (width 0.1524) (layer B.Cu) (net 3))
 (segment (start 158.104 97.73) (end 163.121399 102.747399) (width 0.1524) (layer B.Cu) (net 3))
 (segment (start 190.825001 113.199999) (end 192.025 112) (width 0.1524) (layer F.Cu) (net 5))
 (segment (start 165.129999 113.199999) (end 190.825001 113.199999) (width 0.1524) (layer F.Cu) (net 5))
 (segment (start 162.93 111) (end 165.129999 113.199999) (width 0.1524) (layer F.Cu) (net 5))
 (segment (start 190.800001 96.800001) (end 192 98) (width 0.1524) (layer F.Cu) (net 6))
 (segment (start 165.129999 96.800001) (end 190.800001 96.800001) (width 0.1524) (layer F.Cu) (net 6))
 (segment (start 162.93 99) (end 165.129999 96.800001) (width 0.1524) (layer F.Cu) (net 6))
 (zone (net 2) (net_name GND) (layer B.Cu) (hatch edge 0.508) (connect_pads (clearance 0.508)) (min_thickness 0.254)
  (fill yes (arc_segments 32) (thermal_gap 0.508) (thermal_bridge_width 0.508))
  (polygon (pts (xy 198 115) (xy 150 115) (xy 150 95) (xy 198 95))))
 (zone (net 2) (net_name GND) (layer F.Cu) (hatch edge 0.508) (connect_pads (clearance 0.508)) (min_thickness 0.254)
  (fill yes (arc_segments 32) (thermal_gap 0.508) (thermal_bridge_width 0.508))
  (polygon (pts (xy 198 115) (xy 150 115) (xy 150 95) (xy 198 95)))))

